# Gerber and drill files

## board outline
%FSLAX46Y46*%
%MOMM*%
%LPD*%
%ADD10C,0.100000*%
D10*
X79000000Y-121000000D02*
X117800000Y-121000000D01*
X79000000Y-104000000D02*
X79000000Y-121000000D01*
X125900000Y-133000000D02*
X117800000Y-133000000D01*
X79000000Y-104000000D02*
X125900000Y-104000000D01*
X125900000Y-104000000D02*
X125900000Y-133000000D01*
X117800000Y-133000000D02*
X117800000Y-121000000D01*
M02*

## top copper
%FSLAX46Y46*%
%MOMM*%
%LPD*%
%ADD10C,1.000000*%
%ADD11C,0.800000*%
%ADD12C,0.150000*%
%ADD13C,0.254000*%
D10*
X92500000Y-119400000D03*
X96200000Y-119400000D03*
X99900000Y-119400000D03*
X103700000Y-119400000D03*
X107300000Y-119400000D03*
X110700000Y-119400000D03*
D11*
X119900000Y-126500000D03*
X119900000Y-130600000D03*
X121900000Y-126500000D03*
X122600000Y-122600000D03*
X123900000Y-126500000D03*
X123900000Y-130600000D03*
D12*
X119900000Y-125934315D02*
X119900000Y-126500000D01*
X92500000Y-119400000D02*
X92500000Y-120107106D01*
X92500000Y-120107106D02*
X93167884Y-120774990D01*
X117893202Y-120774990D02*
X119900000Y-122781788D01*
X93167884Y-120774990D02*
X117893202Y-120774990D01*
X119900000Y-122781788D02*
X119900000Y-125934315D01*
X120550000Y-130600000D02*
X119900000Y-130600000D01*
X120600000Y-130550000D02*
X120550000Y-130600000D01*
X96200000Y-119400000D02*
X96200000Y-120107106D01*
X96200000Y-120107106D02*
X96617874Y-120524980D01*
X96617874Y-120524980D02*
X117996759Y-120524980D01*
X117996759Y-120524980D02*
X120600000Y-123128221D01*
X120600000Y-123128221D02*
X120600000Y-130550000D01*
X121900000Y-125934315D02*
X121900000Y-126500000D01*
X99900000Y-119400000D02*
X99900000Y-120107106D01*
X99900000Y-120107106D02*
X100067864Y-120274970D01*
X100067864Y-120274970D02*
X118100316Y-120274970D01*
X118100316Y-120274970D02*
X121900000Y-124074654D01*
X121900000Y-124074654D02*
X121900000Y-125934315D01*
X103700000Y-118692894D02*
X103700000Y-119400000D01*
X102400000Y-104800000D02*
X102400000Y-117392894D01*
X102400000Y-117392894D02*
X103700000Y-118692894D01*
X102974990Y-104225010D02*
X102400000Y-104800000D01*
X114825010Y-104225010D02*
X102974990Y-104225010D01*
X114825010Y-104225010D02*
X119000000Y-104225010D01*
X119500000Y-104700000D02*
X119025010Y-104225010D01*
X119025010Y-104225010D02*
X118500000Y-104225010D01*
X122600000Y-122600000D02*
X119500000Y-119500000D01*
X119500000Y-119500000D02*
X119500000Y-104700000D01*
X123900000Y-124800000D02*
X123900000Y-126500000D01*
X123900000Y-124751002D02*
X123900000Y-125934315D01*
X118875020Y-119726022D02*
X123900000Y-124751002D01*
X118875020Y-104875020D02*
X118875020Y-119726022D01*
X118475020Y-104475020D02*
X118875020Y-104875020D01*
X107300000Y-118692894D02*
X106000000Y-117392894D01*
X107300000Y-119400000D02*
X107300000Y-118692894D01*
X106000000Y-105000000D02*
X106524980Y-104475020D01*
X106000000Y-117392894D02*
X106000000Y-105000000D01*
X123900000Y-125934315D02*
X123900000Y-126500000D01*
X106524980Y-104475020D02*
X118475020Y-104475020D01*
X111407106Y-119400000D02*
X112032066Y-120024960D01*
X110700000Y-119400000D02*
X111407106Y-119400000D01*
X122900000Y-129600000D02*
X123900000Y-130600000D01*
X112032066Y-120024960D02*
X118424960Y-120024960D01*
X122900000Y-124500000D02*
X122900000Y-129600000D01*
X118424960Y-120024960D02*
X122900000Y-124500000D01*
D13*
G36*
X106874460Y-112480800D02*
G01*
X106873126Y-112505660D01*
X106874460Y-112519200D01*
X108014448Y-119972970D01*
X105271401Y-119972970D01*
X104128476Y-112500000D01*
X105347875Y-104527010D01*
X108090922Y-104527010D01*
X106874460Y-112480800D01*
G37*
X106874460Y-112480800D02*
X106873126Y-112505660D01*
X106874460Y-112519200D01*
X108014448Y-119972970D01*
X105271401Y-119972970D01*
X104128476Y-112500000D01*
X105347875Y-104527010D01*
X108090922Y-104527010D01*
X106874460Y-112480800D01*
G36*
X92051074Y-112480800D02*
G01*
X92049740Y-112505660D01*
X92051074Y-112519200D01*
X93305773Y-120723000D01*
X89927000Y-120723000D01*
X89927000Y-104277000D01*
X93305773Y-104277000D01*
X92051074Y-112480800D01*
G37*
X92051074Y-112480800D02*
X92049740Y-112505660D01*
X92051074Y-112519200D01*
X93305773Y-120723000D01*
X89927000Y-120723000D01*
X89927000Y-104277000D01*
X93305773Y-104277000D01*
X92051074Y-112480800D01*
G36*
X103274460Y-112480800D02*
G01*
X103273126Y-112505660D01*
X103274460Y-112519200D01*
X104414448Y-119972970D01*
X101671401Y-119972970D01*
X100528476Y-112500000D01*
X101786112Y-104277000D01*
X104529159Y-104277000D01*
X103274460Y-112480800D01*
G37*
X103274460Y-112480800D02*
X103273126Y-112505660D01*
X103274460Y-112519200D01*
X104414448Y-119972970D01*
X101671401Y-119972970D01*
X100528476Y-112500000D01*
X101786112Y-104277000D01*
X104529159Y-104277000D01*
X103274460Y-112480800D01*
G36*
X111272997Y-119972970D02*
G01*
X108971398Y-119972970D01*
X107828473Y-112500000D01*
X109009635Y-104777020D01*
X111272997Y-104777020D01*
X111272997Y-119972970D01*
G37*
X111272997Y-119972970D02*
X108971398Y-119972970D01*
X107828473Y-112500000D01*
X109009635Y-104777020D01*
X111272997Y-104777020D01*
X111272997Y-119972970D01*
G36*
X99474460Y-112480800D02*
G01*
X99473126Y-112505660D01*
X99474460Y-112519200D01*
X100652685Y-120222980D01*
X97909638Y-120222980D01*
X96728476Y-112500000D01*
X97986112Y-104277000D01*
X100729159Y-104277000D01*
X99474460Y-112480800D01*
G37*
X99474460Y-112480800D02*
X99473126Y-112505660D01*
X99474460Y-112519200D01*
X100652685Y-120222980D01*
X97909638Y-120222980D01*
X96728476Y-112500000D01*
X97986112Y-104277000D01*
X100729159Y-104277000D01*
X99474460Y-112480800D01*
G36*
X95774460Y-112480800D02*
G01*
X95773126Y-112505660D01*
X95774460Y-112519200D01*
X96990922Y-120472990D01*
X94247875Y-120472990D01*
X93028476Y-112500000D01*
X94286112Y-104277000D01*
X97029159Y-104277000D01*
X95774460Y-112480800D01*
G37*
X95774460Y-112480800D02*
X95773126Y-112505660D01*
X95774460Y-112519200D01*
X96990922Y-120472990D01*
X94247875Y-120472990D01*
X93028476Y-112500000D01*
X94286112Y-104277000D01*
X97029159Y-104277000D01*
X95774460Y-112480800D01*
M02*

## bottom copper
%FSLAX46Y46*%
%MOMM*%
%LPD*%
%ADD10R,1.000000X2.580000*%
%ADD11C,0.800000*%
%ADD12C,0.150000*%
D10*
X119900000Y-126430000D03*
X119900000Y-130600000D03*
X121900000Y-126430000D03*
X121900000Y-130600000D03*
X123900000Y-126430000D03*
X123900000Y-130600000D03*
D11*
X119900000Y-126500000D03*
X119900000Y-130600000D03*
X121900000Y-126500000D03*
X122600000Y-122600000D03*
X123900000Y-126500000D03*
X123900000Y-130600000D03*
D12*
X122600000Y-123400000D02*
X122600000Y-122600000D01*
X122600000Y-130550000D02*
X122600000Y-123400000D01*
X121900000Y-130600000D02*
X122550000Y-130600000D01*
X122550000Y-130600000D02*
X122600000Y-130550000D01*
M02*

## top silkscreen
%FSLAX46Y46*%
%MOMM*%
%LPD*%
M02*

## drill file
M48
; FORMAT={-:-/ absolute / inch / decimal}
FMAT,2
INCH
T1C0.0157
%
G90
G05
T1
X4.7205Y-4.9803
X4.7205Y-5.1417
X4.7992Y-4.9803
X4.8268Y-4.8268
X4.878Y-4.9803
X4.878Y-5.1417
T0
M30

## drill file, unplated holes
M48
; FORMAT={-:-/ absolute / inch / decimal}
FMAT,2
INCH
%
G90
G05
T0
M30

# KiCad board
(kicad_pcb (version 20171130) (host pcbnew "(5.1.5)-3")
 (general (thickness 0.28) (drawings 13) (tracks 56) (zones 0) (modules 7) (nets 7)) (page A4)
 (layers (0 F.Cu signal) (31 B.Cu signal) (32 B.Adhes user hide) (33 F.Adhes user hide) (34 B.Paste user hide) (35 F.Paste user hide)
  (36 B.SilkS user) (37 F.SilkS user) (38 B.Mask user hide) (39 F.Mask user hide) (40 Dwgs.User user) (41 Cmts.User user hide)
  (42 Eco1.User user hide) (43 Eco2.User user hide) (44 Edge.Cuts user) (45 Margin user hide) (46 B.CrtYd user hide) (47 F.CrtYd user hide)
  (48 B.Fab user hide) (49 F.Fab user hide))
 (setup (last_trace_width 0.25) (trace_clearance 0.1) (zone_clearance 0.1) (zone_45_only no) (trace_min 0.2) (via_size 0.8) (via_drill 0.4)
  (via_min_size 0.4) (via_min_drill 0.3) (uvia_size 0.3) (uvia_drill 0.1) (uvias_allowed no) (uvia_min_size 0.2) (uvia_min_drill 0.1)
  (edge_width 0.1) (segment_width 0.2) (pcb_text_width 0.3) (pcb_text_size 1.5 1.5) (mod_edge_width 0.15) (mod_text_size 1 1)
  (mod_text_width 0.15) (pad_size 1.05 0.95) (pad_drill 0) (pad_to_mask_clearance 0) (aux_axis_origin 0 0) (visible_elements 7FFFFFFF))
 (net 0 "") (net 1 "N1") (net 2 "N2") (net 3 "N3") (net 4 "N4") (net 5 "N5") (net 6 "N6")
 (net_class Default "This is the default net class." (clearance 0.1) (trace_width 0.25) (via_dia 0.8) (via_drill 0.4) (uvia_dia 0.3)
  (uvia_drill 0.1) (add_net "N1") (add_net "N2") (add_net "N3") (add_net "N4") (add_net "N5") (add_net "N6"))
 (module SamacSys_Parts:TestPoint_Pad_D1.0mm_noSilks (layer F.Cu) (at 92.5 119.4)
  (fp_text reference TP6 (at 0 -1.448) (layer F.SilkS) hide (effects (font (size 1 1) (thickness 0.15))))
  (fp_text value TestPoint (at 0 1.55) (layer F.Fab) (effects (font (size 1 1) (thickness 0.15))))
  (pad 1 smd circle (at 0 0) (size 1 1) (layers F.Cu F.Mask) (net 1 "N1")))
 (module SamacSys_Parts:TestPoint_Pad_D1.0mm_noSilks (layer F.Cu) (at 96.2 119.4)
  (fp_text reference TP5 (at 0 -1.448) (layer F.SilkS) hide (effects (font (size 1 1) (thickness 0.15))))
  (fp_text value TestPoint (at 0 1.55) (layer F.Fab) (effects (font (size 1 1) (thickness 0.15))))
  (pad 1 smd circle (at 0 0) (size 1 1) (layers F.Cu F.Mask) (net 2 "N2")))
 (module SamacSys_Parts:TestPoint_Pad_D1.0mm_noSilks (layer F.Cu) (at 99.9 119.4)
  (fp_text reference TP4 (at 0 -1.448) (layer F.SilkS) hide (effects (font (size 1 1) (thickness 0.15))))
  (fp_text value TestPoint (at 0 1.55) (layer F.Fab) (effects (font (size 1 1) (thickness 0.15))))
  (pad 1 smd circle (at 0 0) (size 1 1) (layers F.Cu F.Mask) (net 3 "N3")))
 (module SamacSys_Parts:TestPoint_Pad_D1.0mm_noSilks (layer F.Cu) (at 103.7 119.4)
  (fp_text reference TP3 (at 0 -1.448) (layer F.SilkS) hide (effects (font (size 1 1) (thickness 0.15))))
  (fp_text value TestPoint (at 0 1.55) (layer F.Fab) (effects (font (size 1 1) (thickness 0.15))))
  (pad 1 smd circle (at 0 0) (size 1 1) (layers F.Cu F.Mask) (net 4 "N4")))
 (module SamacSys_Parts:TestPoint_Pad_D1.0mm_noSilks (layer F.Cu) (at 107.3 119.4)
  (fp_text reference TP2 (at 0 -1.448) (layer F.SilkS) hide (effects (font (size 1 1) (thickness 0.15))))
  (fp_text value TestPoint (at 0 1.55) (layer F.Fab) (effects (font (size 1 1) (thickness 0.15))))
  (pad 1 smd circle (at 0 0) (size 1 1) (layers F.Cu F.Mask) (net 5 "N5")))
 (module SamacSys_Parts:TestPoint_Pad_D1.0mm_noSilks (layer F.Cu) (at 110.7 119.4)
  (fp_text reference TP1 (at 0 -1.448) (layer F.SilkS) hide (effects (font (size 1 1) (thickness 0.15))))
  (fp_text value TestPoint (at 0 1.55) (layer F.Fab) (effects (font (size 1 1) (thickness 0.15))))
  (pad 1 smd circle (at 0 0) (size 1 1) (layers F.Cu F.Mask) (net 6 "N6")))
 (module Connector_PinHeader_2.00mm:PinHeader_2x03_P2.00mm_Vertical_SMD (layer B.Cu) (at 121.9 128.515 270)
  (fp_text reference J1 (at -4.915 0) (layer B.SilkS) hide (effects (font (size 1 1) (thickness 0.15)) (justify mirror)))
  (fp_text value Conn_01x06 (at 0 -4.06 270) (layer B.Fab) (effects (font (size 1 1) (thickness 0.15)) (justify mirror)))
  (pad 1 smd rect (at -2.085 2 270) (size 2.58 1) (layers B.Cu B.Paste B.Mask) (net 1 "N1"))
  (pad 2 smd rect (at 2.085 2 270) (size 2.58 1) (layers B.Cu B.Paste B.Mask) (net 2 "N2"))
  (pad 3 smd rect (at -2.085 0 270) (size 2.58 1) (layers B.Cu B.Paste B.Mask) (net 3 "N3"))
  (pad 4 smd rect (at 2.085 0 270) (size 2.58 1) (layers B.Cu B.Paste B.Mask) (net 4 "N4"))
  (pad 5 smd rect (at -2.085 -2 270) (size 2.58 1) (layers B.Cu B.Paste B.Mask) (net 5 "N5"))
  (pad 6 smd rect (at 2.085 -2 270) (size 2.58 1) (layers B.Cu B.Paste B.Mask) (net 6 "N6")))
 (gr_line (start 79 121) (end 117.8 121) (layer Edge.Cuts) (width 0.1))
 (gr_line (start 79 104) (end 79 121) (layer Edge.Cuts) (width 0.1))
 (gr_line (start 125.9 133) (end 117.8 133) (layer Edge.Cuts) (width 0.1))
 (gr_line (start 79 104) (end 125.9 104) (layer Edge.Cuts) (width 0.1))
 (gr_line (start 125.9 104) (end 125.9 133) (layer Edge.Cuts) (width 0.1))
 (gr_line (start 117.8 133) (end 117.8 121) (layer Edge.Cuts) (width 0.1))
 (via (at 119.9 126.5) (size 0.8) (drill 0.4) (layers F.Cu B.Cu) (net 1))
 (segment (start 119.9 125.934315) (end 119.9 126.5) (width 0.15) (layer F.Cu) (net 1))
 (segment (start 92.5 119.4) (end 92.5 120.107106) (width 0.15) (layer F.Cu) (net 1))
 (segment (start 92.5 120.107106) (end 93.167884 120.77499) (width 0.15) (layer F.Cu) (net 1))
 (segment (start 117.893202 120.77499) (end 119.9 122.781788) (width 0.15) (layer F.Cu) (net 1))
 (segment (start 93.167884 120.77499) (end 117.893202 120.77499) (width 0.15) (layer F.Cu) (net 1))
 (segment (start 119.9 122.781788) (end 119.9 125.934315) (width 0.15) (layer F.Cu) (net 1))
 (via (at 119.9 130.6) (size 0.8) (drill 0.4) (layers F.Cu B.Cu) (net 2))
 (segment (start 120.55 130.6) (end 119.9 130.6) (width 0.15) (layer F.Cu) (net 2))
 (segment (start 120.6 130.55) (end 120.55 130.6) (width 0.15) (layer F.Cu) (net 2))
 (segment (start 96.2 119.4) (end 96.2 120.107106) (width 0.15) (layer F.Cu) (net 2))
 (segment (start 96.2 120.107106) (end 96.617874 120.52498) (width 0.15) (layer F.Cu) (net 2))
 (segment (start 96.617874 120.52498) (end 117.996759 120.52498) (width 0.15) (layer F.Cu) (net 2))
 (segment (start 117.996759 120.52498) (end 120.6 123.128221) (width 0.15) (layer F.Cu) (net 2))
 (segment (start 120.6 123.128221) (end 120.6 130.55) (width 0.15) (layer F.Cu) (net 2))
 (via (at 121.9 126.5) (size 0.8) (drill 0.4) (layers F.Cu B.Cu) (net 3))
 (segment (start 121.9 125.934315) (end 121.9 126.5) (width 0.15) (layer F.Cu) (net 3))
 (segment (start 99.9 119.4) (end 99.9 120.107106) (width 0.15) (layer F.Cu) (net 3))
 (segment (start 99.9 120.107106) (end 100.067864 120.27497) (width 0.15) (layer F.Cu) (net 3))
 (segment (start 100.067864 120.27497) (end 118.100316 120.27497) (width 0.15) (layer F.Cu) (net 3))
 (segment (start 118.100316 120.27497) (end 121.9 124.074654) (width 0.15) (layer F.Cu) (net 3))
 (segment (start 121.9 124.074654) (end 121.9 125.934315) (width 0.15) (layer F.Cu) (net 3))
 (via (at 122.6 122.6) (size 0.8) (drill 0.4) (layers F.Cu B.Cu) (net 4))
 (segment (start 122.6 123.4) (end 122.6 122.6) (width 0.15) (layer B.Cu) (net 4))
 (segment (start 122.6 130.55) (end 122.6 123.4) (width 0.15) (layer B.Cu) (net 4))
 (segment (start 121.9 130.6) (end 122.55 130.6) (width 0.15) (layer B.Cu) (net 4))
 (segment (start 122.55 130.6) (end 122.6 130.55) (width 0.15) (layer B.Cu) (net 4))
 (segment (start 103.7 118.692894) (end 103.7 119.4) (width 0.15) (layer F.Cu) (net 4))
 (segment (start 102.4 104.8) (end 102.4 117.392894) (width 0.15) (layer F.Cu) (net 4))
 (segment (start 102.4 117.392894) (end 103.7 118.692894) (width 0.15) (layer F.Cu) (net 4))
 (segment (start 102.97499 104.22501) (end 102.4 104.8) (width 0.15) (layer F.Cu) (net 4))
 (segment (start 114.82501 104.22501) (end 102.97499 104.22501) (width 0.15) (layer F.Cu) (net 4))
 (segment (start 114.82501 104.22501) (end 119 104.22501) (width 0.15) (layer F.Cu) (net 4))
 (segment (start 119.5 104.7) (end 119.02501 104.22501) (width 0.15) (layer F.Cu) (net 4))
 (segment (start 119.02501 104.22501) (end 118.5 104.22501) (width 0.15) (layer F.Cu) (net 4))
 (segment (start 122.6 122.6) (end 119.5 119.5) (width 0.15) (layer F.Cu) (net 4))
 (segment (start 119.5 119.5) (end 119.5 104.7) (width 0.15) (layer F.Cu) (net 4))
 (via (at 123.9 126.5) (size 0.8) (drill 0.4) (layers F.Cu B.Cu) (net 5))
 (segment (start 123.9 124.8) (end 123.9 126.5) (width 0.15) (layer F.Cu) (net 5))
 (segment (start 123.9 124.751002) (end 123.9 125.934315) (width 0.15) (layer F.Cu) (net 5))
 (segment (start 118.87502 119.726022) (end 123.9 124.751002) (width 0.15) (layer F.Cu) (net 5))
 (segment (start 118.87502 104.87502) (end 118.87502 119.726022) (width 0.15) (layer F.Cu) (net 5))
 (segment (start 118.47502 104.47502) (end 118.87502 104.87502) (width 0.15) (layer F.Cu) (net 5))
 (segment (start 107.3 118.692894) (end 106 117.392894) (width 0.15) (layer F.Cu) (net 5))
 (segment (start 107.3 119.4) (end 107.3 118.692894) (width 0.15) (layer F.Cu) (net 5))
 (segment (start 106 105) (end 106.52498 104.47502) (width 0.15) (layer F.Cu) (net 5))
 (segment (start 106 117.392894) (end 106 105) (width 0.15) (layer F.Cu) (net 5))
 (segment (start 123.9 125.934315) (end 123.9 126.5) (width 0.15) (layer F.Cu) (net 5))
 (segment (start 106.52498 104.47502) (end 118.47502 104.47502) (width 0.15) (layer F.Cu) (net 5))
 (via (at 123.9 130.6) (size 0.8) (drill 0.4) (layers F.Cu B.Cu) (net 6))
 (segment (start 111.407106 119.4) (end 112.032066 120.02496) (width 0.15) (layer F.Cu) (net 6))
 (segment (start 110.7 119.4) (end 111.407106 119.4) (width 0.15) (layer F.Cu) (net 6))
 (segment (start 122.9 129.6) (end 123.9 130.6) (width 0.15) (layer F.Cu) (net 6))
 (segment (start 112.032066 120.02496) (end 118.42496 120.02496) (width 0.15) (layer F.Cu) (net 6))
 (segment (start 122.9 124.5) (end 122.9 129.6) (width 0.15) (layer F.Cu) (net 6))
 (segment (start 118.42496 120.02496) (end 122.9 124.5) (width 0.15) (layer F.Cu) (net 6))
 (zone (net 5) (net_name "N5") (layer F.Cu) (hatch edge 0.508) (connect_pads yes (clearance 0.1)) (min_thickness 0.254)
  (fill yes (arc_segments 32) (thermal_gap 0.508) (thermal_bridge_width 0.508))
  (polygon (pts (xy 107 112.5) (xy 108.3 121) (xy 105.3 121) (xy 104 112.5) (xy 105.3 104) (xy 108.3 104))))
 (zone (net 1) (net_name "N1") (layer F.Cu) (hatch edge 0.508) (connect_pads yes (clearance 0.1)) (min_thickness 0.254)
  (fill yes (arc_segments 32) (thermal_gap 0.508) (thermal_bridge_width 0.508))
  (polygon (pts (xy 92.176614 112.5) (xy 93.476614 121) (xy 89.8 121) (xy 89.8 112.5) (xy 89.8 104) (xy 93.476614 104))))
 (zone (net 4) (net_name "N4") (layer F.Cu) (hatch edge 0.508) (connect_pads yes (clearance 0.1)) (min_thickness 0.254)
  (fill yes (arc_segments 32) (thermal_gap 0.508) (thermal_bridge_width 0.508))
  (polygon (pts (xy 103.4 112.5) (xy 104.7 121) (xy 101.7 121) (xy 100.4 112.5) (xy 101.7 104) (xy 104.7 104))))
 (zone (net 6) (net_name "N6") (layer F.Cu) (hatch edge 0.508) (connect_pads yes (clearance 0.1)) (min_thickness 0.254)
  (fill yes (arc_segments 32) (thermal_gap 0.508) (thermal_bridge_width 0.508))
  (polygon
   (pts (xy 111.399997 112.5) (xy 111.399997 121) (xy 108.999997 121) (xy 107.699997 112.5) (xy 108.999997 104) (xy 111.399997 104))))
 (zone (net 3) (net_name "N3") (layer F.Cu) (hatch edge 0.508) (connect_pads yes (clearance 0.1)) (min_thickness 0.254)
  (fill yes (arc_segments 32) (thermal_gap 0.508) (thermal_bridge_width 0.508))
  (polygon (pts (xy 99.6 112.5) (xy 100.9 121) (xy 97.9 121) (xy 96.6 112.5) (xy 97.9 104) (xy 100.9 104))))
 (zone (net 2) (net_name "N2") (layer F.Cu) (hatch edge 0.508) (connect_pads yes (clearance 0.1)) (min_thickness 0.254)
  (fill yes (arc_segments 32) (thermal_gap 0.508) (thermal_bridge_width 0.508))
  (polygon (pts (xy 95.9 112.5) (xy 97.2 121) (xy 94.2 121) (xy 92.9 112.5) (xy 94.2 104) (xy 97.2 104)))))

